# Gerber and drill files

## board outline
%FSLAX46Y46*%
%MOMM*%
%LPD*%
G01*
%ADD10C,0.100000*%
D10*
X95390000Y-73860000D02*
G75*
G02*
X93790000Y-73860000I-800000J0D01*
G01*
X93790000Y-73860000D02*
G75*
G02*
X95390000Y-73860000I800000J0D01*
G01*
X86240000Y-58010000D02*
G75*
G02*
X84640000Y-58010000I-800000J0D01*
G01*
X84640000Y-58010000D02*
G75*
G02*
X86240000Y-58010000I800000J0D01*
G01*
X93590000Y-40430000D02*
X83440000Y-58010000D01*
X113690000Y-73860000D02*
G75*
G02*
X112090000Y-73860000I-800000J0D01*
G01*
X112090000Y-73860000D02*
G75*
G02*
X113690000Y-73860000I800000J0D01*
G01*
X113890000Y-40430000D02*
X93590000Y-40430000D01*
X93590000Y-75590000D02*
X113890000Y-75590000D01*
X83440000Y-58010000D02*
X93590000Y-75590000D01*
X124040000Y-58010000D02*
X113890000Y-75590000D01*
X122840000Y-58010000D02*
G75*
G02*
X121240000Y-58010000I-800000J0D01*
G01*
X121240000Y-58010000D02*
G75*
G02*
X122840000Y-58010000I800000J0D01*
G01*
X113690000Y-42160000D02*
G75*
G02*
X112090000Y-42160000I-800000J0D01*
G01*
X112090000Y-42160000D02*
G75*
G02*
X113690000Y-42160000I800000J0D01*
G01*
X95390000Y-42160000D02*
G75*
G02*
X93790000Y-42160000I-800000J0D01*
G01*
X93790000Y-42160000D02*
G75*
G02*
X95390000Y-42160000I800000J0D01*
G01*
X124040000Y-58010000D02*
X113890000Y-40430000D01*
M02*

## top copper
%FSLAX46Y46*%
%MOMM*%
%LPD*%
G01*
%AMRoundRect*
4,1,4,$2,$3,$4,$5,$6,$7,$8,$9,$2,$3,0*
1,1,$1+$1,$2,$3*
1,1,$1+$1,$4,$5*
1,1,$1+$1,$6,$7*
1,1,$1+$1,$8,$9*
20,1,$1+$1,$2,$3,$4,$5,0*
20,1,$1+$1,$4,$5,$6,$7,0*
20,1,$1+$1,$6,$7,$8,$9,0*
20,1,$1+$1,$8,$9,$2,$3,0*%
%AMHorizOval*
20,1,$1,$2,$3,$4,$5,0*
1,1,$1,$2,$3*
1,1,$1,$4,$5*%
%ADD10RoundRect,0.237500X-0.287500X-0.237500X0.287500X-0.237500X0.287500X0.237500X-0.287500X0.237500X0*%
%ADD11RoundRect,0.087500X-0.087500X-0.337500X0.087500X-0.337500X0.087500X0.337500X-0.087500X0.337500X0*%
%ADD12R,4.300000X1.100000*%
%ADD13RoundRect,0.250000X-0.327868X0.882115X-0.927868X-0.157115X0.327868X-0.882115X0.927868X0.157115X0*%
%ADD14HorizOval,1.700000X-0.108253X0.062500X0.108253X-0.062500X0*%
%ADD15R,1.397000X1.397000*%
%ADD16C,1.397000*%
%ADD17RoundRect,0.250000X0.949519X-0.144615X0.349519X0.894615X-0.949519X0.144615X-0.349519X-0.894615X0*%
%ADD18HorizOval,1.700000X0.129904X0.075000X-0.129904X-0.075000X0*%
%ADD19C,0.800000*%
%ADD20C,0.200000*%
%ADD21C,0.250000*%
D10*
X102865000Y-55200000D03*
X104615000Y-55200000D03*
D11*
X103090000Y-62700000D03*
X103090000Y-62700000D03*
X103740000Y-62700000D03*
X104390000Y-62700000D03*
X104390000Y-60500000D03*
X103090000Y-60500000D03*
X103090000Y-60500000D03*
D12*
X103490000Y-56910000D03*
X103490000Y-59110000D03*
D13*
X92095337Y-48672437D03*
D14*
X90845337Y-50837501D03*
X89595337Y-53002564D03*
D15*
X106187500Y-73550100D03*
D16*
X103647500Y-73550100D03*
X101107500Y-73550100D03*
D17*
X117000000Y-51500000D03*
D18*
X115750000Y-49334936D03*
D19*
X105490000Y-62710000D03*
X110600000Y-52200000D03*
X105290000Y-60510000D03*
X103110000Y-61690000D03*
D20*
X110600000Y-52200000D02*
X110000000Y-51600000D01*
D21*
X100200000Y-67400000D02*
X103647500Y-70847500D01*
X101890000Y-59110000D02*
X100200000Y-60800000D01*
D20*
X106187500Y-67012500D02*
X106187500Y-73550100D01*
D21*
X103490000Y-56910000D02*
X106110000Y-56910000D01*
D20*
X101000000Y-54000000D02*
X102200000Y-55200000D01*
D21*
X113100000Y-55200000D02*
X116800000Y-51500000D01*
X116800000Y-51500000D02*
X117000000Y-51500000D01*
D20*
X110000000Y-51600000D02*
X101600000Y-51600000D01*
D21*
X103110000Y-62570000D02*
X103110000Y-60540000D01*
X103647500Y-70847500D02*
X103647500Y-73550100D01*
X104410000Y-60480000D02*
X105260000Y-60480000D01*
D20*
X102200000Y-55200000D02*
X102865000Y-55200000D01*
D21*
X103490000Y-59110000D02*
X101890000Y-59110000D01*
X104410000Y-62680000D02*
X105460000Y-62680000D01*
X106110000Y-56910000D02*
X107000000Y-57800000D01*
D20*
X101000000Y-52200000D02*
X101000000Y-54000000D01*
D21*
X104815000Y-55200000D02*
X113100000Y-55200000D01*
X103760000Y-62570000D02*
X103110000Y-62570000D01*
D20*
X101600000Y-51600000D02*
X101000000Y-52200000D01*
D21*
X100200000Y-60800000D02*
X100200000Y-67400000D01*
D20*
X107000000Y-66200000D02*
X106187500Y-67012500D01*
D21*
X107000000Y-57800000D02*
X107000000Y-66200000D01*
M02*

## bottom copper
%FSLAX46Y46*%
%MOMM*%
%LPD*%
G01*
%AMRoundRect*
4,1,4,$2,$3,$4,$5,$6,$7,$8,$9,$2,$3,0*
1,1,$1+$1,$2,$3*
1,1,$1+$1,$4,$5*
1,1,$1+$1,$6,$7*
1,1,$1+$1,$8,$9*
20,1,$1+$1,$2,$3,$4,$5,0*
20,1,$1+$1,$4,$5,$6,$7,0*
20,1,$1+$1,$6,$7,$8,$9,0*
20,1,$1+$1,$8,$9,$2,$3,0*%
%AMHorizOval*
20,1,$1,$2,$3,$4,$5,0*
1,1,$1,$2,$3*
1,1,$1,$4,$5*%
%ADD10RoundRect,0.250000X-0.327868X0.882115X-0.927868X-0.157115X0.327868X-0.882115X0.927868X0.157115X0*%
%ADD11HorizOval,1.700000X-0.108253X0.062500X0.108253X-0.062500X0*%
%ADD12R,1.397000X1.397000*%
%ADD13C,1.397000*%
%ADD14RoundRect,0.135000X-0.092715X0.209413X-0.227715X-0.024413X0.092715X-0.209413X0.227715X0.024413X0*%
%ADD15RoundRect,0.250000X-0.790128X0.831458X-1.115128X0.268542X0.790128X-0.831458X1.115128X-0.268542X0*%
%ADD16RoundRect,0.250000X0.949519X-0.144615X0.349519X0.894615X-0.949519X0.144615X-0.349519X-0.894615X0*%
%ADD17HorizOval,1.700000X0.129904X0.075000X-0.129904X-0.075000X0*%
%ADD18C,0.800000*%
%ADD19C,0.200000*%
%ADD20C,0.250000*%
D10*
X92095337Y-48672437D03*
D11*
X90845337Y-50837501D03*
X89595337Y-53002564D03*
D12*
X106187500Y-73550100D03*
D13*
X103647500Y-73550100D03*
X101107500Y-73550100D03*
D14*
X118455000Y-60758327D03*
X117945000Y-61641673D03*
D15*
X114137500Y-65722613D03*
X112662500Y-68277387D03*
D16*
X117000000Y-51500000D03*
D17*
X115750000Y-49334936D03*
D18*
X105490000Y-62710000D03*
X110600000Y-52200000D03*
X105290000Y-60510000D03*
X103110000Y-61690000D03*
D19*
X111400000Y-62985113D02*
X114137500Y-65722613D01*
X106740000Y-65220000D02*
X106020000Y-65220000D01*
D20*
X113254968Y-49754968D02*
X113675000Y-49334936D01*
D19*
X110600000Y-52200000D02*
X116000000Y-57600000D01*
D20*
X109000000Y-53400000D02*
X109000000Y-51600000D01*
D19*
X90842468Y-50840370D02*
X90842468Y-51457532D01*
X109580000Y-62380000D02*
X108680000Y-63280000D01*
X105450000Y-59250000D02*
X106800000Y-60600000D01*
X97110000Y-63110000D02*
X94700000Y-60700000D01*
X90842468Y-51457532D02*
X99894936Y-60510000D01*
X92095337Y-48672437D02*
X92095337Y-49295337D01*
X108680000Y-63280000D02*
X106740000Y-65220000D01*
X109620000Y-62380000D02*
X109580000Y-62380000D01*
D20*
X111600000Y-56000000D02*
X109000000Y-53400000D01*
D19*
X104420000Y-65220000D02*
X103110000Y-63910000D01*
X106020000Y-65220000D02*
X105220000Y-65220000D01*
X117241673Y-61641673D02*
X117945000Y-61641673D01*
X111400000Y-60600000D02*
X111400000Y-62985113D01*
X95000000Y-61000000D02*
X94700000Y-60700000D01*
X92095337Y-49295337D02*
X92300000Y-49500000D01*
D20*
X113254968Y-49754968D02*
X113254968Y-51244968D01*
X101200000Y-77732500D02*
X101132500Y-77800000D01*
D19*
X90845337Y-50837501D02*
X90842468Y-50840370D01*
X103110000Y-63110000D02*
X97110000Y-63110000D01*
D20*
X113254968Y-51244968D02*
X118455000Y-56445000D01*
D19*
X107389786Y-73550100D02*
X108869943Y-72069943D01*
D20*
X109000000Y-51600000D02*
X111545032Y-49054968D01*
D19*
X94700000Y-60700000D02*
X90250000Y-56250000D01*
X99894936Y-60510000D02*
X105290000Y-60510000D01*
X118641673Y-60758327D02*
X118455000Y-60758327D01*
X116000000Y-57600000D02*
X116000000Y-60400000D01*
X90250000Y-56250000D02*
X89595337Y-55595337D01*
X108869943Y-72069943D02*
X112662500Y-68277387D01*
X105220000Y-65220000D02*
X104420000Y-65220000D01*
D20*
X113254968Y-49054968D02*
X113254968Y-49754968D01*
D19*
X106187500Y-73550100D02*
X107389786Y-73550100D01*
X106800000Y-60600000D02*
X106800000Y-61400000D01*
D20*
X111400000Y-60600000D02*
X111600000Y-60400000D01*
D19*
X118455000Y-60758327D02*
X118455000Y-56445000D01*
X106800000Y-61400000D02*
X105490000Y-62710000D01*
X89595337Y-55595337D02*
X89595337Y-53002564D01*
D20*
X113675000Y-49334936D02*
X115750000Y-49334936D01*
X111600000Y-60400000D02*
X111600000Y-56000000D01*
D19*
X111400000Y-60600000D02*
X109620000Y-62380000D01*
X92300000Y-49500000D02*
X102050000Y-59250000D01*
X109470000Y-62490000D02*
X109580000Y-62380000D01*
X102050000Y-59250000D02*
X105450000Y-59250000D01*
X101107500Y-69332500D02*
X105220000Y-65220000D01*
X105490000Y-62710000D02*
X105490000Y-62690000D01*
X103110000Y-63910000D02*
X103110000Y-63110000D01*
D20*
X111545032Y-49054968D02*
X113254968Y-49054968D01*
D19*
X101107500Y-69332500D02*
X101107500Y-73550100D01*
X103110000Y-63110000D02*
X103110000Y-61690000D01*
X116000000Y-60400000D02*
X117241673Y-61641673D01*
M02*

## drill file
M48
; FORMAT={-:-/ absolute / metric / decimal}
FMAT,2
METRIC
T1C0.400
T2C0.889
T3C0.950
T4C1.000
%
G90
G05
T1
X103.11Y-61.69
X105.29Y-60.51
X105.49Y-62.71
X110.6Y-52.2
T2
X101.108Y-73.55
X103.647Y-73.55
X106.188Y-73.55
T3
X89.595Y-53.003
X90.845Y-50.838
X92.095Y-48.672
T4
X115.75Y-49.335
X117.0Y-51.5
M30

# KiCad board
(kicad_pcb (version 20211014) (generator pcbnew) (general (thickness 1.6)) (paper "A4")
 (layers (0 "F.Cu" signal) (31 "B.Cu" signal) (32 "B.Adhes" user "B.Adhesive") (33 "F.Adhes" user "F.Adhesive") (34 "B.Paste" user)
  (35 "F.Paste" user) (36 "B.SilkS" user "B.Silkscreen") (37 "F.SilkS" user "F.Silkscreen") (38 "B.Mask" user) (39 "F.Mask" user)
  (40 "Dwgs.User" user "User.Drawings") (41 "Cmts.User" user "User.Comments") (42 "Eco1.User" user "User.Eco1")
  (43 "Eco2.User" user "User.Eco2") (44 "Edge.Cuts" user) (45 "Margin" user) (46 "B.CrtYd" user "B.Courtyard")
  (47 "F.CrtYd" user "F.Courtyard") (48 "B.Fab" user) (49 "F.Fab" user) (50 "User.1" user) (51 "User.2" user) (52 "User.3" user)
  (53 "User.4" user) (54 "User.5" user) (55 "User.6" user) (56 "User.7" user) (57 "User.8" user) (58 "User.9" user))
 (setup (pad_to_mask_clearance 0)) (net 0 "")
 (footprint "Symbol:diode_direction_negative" (layer "F.Cu") (at 103.8 52.65)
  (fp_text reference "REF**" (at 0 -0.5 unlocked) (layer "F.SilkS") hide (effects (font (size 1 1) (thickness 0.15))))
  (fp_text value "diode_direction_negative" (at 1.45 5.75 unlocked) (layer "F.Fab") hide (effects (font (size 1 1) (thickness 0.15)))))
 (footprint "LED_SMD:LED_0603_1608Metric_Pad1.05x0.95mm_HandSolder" (layer "F.Cu") (at 103.74 55.2)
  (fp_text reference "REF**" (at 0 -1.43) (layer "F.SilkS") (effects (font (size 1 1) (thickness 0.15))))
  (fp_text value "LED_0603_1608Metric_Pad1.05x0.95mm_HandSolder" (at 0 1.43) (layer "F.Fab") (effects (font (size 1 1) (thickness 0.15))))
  (pad "1" smd roundrect (at -0.875 0) (size 1.05 0.95) (layers "F.Cu" "F.Paste" "F.Mask") (roundrect_rratio 0.25))
  (pad "2" smd roundrect (at 0.875 0) (size 1.05 0.95) (layers "F.Cu" "F.Paste" "F.Mask") (roundrect_rratio 0.25)))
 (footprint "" (layer "F.Cu") (at 103.09 62.7)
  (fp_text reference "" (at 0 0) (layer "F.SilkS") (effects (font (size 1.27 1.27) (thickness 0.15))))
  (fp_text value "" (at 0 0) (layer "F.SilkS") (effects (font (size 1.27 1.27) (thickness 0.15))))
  (pad "1" smd roundrect (at 0 0) (size 0.35 0.85) (layers "F.Cu" "F.Paste" "F.Mask") (roundrect_rratio 0.25)))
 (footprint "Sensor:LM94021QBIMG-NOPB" (layer "F.Cu") (at 103.74 61.6)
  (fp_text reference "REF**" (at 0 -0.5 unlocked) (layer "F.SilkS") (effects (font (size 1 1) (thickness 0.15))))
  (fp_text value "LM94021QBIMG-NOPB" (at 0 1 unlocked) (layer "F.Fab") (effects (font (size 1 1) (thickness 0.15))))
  (pad "1" smd roundrect (at -0.65 1.1) (size 0.35 0.85) (layers "F.Cu" "F.Paste" "F.Mask") (roundrect_rratio 0.25))
  (pad "2" smd roundrect (at 0 1.1) (size 0.35 0.85) (layers "F.Cu" "F.Paste" "F.Mask") (roundrect_rratio 0.25))
  (pad "3" smd roundrect (at 0.65 1.1) (size 0.35 0.85) (layers "F.Cu" "F.Paste" "F.Mask") (roundrect_rratio 0.25))
  (pad "4" smd roundrect (at 0.65 -1.1) (size 0.35 0.85) (layers "F.Cu" "F.Paste" "F.Mask") (roundrect_rratio 0.25))
  (pad "5" smd roundrect (at -0.65 -1.1) (size 0.35 0.85) (layers "F.Cu" "F.Paste" "F.Mask") (roundrect_rratio 0.25)))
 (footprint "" (layer "F.Cu") (at 103.09 60.5)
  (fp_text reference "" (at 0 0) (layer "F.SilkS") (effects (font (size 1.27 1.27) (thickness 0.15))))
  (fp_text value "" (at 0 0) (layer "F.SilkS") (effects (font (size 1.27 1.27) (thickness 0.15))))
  (pad "5" smd roundrect (at 0 0) (size 0.35 0.85) (layers "F.Cu" "F.Paste" "F.Mask") (roundrect_rratio 0.25)))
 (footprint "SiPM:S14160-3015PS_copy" (layer "F.Cu") (at 103.74 58.01)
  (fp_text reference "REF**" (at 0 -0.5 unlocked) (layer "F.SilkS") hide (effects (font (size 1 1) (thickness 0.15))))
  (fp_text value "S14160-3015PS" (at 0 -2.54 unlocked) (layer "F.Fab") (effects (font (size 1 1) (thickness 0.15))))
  (pad "1" smd rect (at -0.25 -1.1) (size 4.3 1.1) (layers "F.Cu" "F.Paste" "F.Mask"))
  (pad "2" smd rect (at -0.25 1.1) (size 4.3 1.1) (layers "F.Cu" "F.Paste" "F.Mask")))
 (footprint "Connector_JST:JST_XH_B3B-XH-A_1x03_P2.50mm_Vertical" (layer "B.Cu") (at 92.095337 48.672437 -120)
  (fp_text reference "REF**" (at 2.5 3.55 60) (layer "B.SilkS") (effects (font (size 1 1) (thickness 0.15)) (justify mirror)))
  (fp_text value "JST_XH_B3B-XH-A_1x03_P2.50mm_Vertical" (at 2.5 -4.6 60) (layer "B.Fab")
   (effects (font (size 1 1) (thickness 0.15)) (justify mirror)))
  (pad "1" thru_hole roundrect (at 0 0 240) (size 1.7 1.95) (drill 0.95) (layers *.Cu *.Mask) (roundrect_rratio 0.1470588235))
  (pad "2" thru_hole oval (at 2.5 0 240) (size 1.7 1.95) (drill 0.95) (layers *.Cu *.Mask))
  (pad "3" thru_hole oval (at 5 0 240) (size 1.7 1.95) (drill 0.95) (layers *.Cu *.Mask)))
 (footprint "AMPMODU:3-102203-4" (layer "B.Cu") (at 106.1875 73.5501 180)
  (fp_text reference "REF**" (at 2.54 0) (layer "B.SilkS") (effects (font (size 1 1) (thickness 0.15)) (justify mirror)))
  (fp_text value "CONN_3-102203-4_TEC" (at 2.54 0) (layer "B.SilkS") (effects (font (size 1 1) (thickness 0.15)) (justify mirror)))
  (pad "1" thru_hole rect locked (at 0 0 180) (size 1.397 1.397) (drill 0.889) (layers *.Cu *.Mask))
  (pad "2" thru_hole circle locked (at 2.54 0 180) (size 1.397 1.397) (drill 0.889) (layers *.Cu *.Mask))
  (pad "3" thru_hole circle locked (at 5.08 0 180) (size 1.397 1.397) (drill 0.889) (layers *.Cu *.Mask)))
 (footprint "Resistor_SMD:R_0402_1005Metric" (layer "B.Cu") (at 118.2 61.2 -120)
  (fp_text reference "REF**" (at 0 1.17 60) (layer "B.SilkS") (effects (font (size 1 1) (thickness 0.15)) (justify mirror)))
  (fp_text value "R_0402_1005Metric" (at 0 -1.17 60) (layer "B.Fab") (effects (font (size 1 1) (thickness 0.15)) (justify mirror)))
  (pad "1" smd roundrect (at -0.51 0 240) (size 0.54 0.64) (layers "B.Cu" "B.Paste" "B.Mask") (roundrect_rratio 0.25))
  (pad "2" smd roundrect (at 0.51 0 240) (size 0.54 0.64) (layers "B.Cu" "B.Paste" "B.Mask") (roundrect_rratio 0.25)))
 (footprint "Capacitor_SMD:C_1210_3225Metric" (layer "B.Cu") (at 113.4 67 -120)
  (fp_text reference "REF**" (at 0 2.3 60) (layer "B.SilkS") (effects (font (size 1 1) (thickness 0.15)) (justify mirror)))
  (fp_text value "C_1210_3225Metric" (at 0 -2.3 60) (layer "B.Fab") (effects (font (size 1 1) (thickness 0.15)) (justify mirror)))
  (pad "1" smd roundrect (at -1.475 0 240) (size 1.15 2.7) (layers "B.Cu" "B.Paste" "B.Mask") (roundrect_rratio 0.2173913043))
  (pad "2" smd roundrect (at 1.475 0 240) (size 1.15 2.7) (layers "B.Cu" "B.Paste" "B.Mask") (roundrect_rratio 0.2173913043)))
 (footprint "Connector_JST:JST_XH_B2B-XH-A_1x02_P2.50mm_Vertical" (layer "B.Cu") (at 117 51.5 120)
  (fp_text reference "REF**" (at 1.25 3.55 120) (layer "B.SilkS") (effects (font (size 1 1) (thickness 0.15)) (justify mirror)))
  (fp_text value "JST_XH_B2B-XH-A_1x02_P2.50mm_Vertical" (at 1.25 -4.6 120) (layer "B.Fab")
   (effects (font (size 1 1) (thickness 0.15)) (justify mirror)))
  (pad "1" thru_hole roundrect (at 0 0 120) (size 1.7 2) (drill 1) (layers *.Cu *.Mask) (roundrect_rratio 0.1470588235))
  (pad "2" thru_hole oval (at 2.5 0 120) (size 1.7 2) (drill 1) (layers *.Cu *.Mask)))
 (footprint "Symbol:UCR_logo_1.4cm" (layer "B.Cu") (at 104.4 44.5 180)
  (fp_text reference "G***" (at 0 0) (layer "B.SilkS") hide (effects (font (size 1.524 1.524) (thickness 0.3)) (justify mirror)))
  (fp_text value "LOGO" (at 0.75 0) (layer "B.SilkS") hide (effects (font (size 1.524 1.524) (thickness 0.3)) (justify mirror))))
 (gr_circle (center 94.59 73.86) (end 95.39 73.86) (layer "Edge.Cuts") (width 0.1) (fill none))
 (gr_circle (center 85.44 58.01) (end 86.24 58.01) (layer "Edge.Cuts") (width 0.1) (fill none))
 (gr_line (start 93.59 40.43) (end 83.44 58.01) (layer "Edge.Cuts") (width 0.1))
 (gr_circle (center 112.89 73.86) (end 113.69 73.86) (layer "Edge.Cuts") (width 0.1) (fill none))
 (gr_line (start 113.89 40.43) (end 93.59 40.43) (layer "Edge.Cuts") (width 0.1))
 (gr_line (start 93.59 75.59) (end 113.89 75.59) (layer "Edge.Cuts") (width 0.1))
 (gr_line (start 83.44 58.01) (end 93.59 75.59) (layer "Edge.Cuts") (width 0.1))
 (gr_line (start 124.04 58.01) (end 113.89 75.59) (layer "Edge.Cuts") (width 0.1))
 (gr_circle (center 122.04 58.01) (end 122.84 58.01) (layer "Edge.Cuts") (width 0.1) (fill none))
 (gr_circle (center 112.89 42.16) (end 113.69 42.16) (layer "Edge.Cuts") (width 0.1) (fill none))
 (gr_circle (center 94.59 42.16) (end 95.39 42.16) (layer "Edge.Cuts") (width 0.1) (fill none))
 (gr_line (start 124.04 58.01) (end 113.89 40.43) (layer "Edge.Cuts") (width 0.1))
 (segment (start 110.6 52.2) (end 110 51.6) (width 0.2) (layer "F.Cu") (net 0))
 (segment (start 100.2 67.4) (end 103.6475 70.8475) (width 0.25) (layer "F.Cu") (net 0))
 (segment (start 101.89 59.11) (end 100.2 60.8) (width 0.25) (layer "F.Cu") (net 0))
 (segment (start 106.1875 67.0125) (end 106.1875 73.5501) (width 0.2) (layer "F.Cu") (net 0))
 (segment (start 103.49 56.91) (end 106.11 56.91) (width 0.25) (layer "F.Cu") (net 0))
 (segment (start 101 54) (end 102.2 55.2) (width 0.2) (layer "F.Cu") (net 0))
 (segment (start 113.1 55.2) (end 116.8 51.5) (width 0.25) (layer "F.Cu") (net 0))
 (segment (start 116.8 51.5) (end 117 51.5) (width 0.25) (layer "F.Cu") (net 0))
 (segment (start 110 51.6) (end 101.6 51.6) (width 0.2) (layer "F.Cu") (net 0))
 (segment (start 103.11 62.57) (end 103.11 60.54) (width 0.25) (layer "F.Cu") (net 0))
 (segment (start 103.6475 70.8475) (end 103.6475 73.5501) (width 0.25) (layer "F.Cu") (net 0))
 (segment (start 104.41 60.48) (end 105.26 60.48) (width 0.25) (layer "F.Cu") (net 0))
 (segment (start 102.2 55.2) (end 102.865 55.2) (width 0.2) (layer "F.Cu") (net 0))
 (segment (start 103.49 59.11) (end 101.89 59.11) (width 0.25) (layer "F.Cu") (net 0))
 (segment (start 104.41 62.68) (end 105.46 62.68) (width 0.25) (layer "F.Cu") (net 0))
 (segment (start 106.11 56.91) (end 107 57.8) (width 0.25) (layer "F.Cu") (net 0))
 (segment (start 101 52.2) (end 101 54) (width 0.2) (layer "F.Cu") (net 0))
 (segment (start 104.815 55.2) (end 113.1 55.2) (width 0.25) (layer "F.Cu") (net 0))
 (segment (start 103.76 62.57) (end 103.11 62.57) (width 0.25) (layer "F.Cu") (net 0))
 (segment (start 101.6 51.6) (end 101 52.2) (width 0.2) (layer "F.Cu") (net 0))
 (segment (start 100.2 60.8) (end 100.2 67.4) (width 0.25) (layer "F.Cu") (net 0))
 (segment (start 107 66.2) (end 106.1875 67.0125) (width 0.2) (layer "F.Cu") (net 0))
 (segment (start 107 57.8) (end 107 66.2) (width 0.25) (layer "F.Cu") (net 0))
 (via (at 105.49 62.71) (size 0.8) (drill 0.4) (layers "F.Cu" "B.Cu") (free) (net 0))
 (via (at 110.6 52.2) (size 0.8) (drill 0.4) (layers "F.Cu" "B.Cu") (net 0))
 (via (at 105.29 60.51) (size 0.8) (drill 0.4) (layers "F.Cu" "B.Cu") (free) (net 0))
 (via (at 103.11 61.69) (size 0.8) (drill 0.4) (layers "F.Cu" "B.Cu") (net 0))
 (segment (start 111.4 62.985113) (end 114.1375 65.722613) (width 0.2) (layer "B.Cu") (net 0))
 (segment (start 106.74 65.22) (end 106.02 65.22) (width 0.2) (layer "B.Cu") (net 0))
 (segment (start 113.254968 49.754968) (end 113.675 49.334936) (width 0.25) (layer "B.Cu") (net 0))
 (segment (start 110.6 52.2) (end 116 57.6) (width 0.2) (layer "B.Cu") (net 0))
 (segment (start 109 53.4) (end 109 51.6) (width 0.25) (layer "B.Cu") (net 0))
 (segment (start 90.842468 50.84037) (end 90.842468 51.457532) (width 0.2) (layer "B.Cu") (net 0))
 (segment (start 109.58 62.38) (end 108.68 63.28) (width 0.2) (layer "B.Cu") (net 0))
 (segment (start 105.45 59.25) (end 106.8 60.6) (width 0.2) (layer "B.Cu") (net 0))
 (segment (start 97.11 63.11) (end 94.7 60.7) (width 0.2) (layer "B.Cu") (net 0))
 (segment (start 90.842468 51.457532) (end 99.894936 60.51) (width 0.2) (layer "B.Cu") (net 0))
 (segment (start 92.095337 48.672437) (end 92.095337 49.295337) (width 0.2) (layer "B.Cu") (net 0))
 (segment (start 108.68 63.28) (end 106.74 65.22) (width 0.2) (layer "B.Cu") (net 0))
 (segment (start 109.62 62.38) (end 109.58 62.38) (width 0.2) (layer "B.Cu") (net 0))
 (segment (start 111.6 56) (end 109 53.4) (width 0.25) (layer "B.Cu") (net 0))
 (segment (start 104.42 65.22) (end 103.11 63.91) (width 0.2) (layer "B.Cu") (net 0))
 (segment (start 106.02 65.22) (end 105.22 65.22) (width 0.2) (layer "B.Cu") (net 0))
 (segment (start 117.241673 61.641673) (end 117.945 61.641673) (width 0.2) (layer "B.Cu") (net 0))
 (segment (start 111.4 60.6) (end 111.4 62.985113) (width 0.2) (layer "B.Cu") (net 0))
 (segment (start 95 61) (end 94.7 60.7) (width 0.2) (layer "B.Cu") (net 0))
 (segment (start 92.095337 49.295337) (end 92.3 49.5) (width 0.2) (layer "B.Cu") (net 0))
 (segment (start 113.254968 49.754968) (end 113.254968 51.244968) (width 0.25) (layer "B.Cu") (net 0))
 (segment (start 101.2 77.7325) (end 101.1325 77.8) (width 0.25) (layer "B.Cu") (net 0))
 (segment (start 90.845337 50.837501) (end 90.842468 50.84037) (width 0.2) (layer "B.Cu") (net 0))
 (segment (start 103.11 63.11) (end 97.11 63.11) (width 0.2) (layer "B.Cu") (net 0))
 (segment (start 113.254968 51.244968) (end 118.455 56.445) (width 0.25) (layer "B.Cu") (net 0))
 (segment (start 107.389786 73.5501) (end 108.869943 72.069943) (width 0.2) (layer "B.Cu") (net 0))
 (segment (start 109 51.6) (end 111.545032 49.054968) (width 0.25) (layer "B.Cu") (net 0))
 (segment (start 94.7 60.7) (end 90.25 56.25) (width 0.2) (layer "B.Cu") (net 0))
 (segment (start 99.894936 60.51) (end 105.29 60.51) (width 0.2) (layer "B.Cu") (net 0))
 (segment (start 118.641673 60.758327) (end 118.455 60.758327) (width 0.2) (layer "B.Cu") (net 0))
 (segment (start 116 57.6) (end 116 60.4) (width 0.2) (layer "B.Cu") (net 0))
 (segment (start 90.25 56.25) (end 89.595337 55.595337) (width 0.2) (layer "B.Cu") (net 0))
 (segment (start 108.869943 72.069943) (end 112.6625 68.277387) (width 0.2) (layer "B.Cu") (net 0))
 (segment (start 105.22 65.22) (end 104.42 65.22) (width 0.2) (layer "B.Cu") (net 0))
 (segment (start 113.254968 49.054968) (end 113.254968 49.754968) (width 0.25) (layer "B.Cu") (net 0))
 (segment (start 106.1875 73.5501) (end 107.389786 73.5501) (width 0.2) (layer "B.Cu") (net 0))
 (segment (start 106.8 60.6) (end 106.8 61.4) (width 0.2) (layer "B.Cu") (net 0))
 (segment (start 111.4 60.6) (end 111.6 60.4) (width 0.25) (layer "B.Cu") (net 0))
 (segment (start 118.455 60.758327) (end 118.455 56.445) (width 0.2) (layer "B.Cu") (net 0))
 (segment (start 106.8 61.4) (end 105.49 62.71) (width 0.2) (layer "B.Cu") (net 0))
 (segment (start 89.595337 55.595337) (end 89.595337 53.002564) (width 0.2) (layer "B.Cu") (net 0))
 (segment (start 113.675 49.334936) (end 115.75 49.334936) (width 0.25) (layer "B.Cu") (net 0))
 (segment (start 111.6 60.4) (end 111.6 56) (width 0.25) (layer "B.Cu") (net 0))
 (segment (start 111.4 60.6) (end 109.62 62.38) (width 0.2) (layer "B.Cu") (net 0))
 (segment (start 92.3 49.5) (end 102.05 59.25) (width 0.2) (layer "B.Cu") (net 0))
 (segment (start 109.47 62.49) (end 109.58 62.38) (width 0.2) (layer "B.Cu") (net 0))
 (segment (start 102.05 59.25) (end 105.45 59.25) (width 0.2) (layer "B.Cu") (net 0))
 (segment (start 101.1075 69.3325) (end 105.22 65.22) (width 0.2) (layer "B.Cu") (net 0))
 (segment (start 105.49 62.71) (end 105.49 62.69) (width 0.2) (layer "B.Cu") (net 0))
 (segment (start 103.11 63.91) (end 103.11 63.11) (width 0.2) (layer "B.Cu") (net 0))
 (segment (start 111.545032 49.054968) (end 113.254968 49.054968) (width 0.25) (layer "B.Cu") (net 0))
 (segment (start 101.1075 69.3325) (end 101.1075 73.5501) (width 0.2) (layer "B.Cu") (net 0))
 (segment (start 103.11 63.11) (end 103.11 61.69) (width 0.2) (layer "B.Cu") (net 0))
 (segment (start 116 60.4) (end 117.241673 61.641673) (width 0.2) (layer "B.Cu") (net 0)))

